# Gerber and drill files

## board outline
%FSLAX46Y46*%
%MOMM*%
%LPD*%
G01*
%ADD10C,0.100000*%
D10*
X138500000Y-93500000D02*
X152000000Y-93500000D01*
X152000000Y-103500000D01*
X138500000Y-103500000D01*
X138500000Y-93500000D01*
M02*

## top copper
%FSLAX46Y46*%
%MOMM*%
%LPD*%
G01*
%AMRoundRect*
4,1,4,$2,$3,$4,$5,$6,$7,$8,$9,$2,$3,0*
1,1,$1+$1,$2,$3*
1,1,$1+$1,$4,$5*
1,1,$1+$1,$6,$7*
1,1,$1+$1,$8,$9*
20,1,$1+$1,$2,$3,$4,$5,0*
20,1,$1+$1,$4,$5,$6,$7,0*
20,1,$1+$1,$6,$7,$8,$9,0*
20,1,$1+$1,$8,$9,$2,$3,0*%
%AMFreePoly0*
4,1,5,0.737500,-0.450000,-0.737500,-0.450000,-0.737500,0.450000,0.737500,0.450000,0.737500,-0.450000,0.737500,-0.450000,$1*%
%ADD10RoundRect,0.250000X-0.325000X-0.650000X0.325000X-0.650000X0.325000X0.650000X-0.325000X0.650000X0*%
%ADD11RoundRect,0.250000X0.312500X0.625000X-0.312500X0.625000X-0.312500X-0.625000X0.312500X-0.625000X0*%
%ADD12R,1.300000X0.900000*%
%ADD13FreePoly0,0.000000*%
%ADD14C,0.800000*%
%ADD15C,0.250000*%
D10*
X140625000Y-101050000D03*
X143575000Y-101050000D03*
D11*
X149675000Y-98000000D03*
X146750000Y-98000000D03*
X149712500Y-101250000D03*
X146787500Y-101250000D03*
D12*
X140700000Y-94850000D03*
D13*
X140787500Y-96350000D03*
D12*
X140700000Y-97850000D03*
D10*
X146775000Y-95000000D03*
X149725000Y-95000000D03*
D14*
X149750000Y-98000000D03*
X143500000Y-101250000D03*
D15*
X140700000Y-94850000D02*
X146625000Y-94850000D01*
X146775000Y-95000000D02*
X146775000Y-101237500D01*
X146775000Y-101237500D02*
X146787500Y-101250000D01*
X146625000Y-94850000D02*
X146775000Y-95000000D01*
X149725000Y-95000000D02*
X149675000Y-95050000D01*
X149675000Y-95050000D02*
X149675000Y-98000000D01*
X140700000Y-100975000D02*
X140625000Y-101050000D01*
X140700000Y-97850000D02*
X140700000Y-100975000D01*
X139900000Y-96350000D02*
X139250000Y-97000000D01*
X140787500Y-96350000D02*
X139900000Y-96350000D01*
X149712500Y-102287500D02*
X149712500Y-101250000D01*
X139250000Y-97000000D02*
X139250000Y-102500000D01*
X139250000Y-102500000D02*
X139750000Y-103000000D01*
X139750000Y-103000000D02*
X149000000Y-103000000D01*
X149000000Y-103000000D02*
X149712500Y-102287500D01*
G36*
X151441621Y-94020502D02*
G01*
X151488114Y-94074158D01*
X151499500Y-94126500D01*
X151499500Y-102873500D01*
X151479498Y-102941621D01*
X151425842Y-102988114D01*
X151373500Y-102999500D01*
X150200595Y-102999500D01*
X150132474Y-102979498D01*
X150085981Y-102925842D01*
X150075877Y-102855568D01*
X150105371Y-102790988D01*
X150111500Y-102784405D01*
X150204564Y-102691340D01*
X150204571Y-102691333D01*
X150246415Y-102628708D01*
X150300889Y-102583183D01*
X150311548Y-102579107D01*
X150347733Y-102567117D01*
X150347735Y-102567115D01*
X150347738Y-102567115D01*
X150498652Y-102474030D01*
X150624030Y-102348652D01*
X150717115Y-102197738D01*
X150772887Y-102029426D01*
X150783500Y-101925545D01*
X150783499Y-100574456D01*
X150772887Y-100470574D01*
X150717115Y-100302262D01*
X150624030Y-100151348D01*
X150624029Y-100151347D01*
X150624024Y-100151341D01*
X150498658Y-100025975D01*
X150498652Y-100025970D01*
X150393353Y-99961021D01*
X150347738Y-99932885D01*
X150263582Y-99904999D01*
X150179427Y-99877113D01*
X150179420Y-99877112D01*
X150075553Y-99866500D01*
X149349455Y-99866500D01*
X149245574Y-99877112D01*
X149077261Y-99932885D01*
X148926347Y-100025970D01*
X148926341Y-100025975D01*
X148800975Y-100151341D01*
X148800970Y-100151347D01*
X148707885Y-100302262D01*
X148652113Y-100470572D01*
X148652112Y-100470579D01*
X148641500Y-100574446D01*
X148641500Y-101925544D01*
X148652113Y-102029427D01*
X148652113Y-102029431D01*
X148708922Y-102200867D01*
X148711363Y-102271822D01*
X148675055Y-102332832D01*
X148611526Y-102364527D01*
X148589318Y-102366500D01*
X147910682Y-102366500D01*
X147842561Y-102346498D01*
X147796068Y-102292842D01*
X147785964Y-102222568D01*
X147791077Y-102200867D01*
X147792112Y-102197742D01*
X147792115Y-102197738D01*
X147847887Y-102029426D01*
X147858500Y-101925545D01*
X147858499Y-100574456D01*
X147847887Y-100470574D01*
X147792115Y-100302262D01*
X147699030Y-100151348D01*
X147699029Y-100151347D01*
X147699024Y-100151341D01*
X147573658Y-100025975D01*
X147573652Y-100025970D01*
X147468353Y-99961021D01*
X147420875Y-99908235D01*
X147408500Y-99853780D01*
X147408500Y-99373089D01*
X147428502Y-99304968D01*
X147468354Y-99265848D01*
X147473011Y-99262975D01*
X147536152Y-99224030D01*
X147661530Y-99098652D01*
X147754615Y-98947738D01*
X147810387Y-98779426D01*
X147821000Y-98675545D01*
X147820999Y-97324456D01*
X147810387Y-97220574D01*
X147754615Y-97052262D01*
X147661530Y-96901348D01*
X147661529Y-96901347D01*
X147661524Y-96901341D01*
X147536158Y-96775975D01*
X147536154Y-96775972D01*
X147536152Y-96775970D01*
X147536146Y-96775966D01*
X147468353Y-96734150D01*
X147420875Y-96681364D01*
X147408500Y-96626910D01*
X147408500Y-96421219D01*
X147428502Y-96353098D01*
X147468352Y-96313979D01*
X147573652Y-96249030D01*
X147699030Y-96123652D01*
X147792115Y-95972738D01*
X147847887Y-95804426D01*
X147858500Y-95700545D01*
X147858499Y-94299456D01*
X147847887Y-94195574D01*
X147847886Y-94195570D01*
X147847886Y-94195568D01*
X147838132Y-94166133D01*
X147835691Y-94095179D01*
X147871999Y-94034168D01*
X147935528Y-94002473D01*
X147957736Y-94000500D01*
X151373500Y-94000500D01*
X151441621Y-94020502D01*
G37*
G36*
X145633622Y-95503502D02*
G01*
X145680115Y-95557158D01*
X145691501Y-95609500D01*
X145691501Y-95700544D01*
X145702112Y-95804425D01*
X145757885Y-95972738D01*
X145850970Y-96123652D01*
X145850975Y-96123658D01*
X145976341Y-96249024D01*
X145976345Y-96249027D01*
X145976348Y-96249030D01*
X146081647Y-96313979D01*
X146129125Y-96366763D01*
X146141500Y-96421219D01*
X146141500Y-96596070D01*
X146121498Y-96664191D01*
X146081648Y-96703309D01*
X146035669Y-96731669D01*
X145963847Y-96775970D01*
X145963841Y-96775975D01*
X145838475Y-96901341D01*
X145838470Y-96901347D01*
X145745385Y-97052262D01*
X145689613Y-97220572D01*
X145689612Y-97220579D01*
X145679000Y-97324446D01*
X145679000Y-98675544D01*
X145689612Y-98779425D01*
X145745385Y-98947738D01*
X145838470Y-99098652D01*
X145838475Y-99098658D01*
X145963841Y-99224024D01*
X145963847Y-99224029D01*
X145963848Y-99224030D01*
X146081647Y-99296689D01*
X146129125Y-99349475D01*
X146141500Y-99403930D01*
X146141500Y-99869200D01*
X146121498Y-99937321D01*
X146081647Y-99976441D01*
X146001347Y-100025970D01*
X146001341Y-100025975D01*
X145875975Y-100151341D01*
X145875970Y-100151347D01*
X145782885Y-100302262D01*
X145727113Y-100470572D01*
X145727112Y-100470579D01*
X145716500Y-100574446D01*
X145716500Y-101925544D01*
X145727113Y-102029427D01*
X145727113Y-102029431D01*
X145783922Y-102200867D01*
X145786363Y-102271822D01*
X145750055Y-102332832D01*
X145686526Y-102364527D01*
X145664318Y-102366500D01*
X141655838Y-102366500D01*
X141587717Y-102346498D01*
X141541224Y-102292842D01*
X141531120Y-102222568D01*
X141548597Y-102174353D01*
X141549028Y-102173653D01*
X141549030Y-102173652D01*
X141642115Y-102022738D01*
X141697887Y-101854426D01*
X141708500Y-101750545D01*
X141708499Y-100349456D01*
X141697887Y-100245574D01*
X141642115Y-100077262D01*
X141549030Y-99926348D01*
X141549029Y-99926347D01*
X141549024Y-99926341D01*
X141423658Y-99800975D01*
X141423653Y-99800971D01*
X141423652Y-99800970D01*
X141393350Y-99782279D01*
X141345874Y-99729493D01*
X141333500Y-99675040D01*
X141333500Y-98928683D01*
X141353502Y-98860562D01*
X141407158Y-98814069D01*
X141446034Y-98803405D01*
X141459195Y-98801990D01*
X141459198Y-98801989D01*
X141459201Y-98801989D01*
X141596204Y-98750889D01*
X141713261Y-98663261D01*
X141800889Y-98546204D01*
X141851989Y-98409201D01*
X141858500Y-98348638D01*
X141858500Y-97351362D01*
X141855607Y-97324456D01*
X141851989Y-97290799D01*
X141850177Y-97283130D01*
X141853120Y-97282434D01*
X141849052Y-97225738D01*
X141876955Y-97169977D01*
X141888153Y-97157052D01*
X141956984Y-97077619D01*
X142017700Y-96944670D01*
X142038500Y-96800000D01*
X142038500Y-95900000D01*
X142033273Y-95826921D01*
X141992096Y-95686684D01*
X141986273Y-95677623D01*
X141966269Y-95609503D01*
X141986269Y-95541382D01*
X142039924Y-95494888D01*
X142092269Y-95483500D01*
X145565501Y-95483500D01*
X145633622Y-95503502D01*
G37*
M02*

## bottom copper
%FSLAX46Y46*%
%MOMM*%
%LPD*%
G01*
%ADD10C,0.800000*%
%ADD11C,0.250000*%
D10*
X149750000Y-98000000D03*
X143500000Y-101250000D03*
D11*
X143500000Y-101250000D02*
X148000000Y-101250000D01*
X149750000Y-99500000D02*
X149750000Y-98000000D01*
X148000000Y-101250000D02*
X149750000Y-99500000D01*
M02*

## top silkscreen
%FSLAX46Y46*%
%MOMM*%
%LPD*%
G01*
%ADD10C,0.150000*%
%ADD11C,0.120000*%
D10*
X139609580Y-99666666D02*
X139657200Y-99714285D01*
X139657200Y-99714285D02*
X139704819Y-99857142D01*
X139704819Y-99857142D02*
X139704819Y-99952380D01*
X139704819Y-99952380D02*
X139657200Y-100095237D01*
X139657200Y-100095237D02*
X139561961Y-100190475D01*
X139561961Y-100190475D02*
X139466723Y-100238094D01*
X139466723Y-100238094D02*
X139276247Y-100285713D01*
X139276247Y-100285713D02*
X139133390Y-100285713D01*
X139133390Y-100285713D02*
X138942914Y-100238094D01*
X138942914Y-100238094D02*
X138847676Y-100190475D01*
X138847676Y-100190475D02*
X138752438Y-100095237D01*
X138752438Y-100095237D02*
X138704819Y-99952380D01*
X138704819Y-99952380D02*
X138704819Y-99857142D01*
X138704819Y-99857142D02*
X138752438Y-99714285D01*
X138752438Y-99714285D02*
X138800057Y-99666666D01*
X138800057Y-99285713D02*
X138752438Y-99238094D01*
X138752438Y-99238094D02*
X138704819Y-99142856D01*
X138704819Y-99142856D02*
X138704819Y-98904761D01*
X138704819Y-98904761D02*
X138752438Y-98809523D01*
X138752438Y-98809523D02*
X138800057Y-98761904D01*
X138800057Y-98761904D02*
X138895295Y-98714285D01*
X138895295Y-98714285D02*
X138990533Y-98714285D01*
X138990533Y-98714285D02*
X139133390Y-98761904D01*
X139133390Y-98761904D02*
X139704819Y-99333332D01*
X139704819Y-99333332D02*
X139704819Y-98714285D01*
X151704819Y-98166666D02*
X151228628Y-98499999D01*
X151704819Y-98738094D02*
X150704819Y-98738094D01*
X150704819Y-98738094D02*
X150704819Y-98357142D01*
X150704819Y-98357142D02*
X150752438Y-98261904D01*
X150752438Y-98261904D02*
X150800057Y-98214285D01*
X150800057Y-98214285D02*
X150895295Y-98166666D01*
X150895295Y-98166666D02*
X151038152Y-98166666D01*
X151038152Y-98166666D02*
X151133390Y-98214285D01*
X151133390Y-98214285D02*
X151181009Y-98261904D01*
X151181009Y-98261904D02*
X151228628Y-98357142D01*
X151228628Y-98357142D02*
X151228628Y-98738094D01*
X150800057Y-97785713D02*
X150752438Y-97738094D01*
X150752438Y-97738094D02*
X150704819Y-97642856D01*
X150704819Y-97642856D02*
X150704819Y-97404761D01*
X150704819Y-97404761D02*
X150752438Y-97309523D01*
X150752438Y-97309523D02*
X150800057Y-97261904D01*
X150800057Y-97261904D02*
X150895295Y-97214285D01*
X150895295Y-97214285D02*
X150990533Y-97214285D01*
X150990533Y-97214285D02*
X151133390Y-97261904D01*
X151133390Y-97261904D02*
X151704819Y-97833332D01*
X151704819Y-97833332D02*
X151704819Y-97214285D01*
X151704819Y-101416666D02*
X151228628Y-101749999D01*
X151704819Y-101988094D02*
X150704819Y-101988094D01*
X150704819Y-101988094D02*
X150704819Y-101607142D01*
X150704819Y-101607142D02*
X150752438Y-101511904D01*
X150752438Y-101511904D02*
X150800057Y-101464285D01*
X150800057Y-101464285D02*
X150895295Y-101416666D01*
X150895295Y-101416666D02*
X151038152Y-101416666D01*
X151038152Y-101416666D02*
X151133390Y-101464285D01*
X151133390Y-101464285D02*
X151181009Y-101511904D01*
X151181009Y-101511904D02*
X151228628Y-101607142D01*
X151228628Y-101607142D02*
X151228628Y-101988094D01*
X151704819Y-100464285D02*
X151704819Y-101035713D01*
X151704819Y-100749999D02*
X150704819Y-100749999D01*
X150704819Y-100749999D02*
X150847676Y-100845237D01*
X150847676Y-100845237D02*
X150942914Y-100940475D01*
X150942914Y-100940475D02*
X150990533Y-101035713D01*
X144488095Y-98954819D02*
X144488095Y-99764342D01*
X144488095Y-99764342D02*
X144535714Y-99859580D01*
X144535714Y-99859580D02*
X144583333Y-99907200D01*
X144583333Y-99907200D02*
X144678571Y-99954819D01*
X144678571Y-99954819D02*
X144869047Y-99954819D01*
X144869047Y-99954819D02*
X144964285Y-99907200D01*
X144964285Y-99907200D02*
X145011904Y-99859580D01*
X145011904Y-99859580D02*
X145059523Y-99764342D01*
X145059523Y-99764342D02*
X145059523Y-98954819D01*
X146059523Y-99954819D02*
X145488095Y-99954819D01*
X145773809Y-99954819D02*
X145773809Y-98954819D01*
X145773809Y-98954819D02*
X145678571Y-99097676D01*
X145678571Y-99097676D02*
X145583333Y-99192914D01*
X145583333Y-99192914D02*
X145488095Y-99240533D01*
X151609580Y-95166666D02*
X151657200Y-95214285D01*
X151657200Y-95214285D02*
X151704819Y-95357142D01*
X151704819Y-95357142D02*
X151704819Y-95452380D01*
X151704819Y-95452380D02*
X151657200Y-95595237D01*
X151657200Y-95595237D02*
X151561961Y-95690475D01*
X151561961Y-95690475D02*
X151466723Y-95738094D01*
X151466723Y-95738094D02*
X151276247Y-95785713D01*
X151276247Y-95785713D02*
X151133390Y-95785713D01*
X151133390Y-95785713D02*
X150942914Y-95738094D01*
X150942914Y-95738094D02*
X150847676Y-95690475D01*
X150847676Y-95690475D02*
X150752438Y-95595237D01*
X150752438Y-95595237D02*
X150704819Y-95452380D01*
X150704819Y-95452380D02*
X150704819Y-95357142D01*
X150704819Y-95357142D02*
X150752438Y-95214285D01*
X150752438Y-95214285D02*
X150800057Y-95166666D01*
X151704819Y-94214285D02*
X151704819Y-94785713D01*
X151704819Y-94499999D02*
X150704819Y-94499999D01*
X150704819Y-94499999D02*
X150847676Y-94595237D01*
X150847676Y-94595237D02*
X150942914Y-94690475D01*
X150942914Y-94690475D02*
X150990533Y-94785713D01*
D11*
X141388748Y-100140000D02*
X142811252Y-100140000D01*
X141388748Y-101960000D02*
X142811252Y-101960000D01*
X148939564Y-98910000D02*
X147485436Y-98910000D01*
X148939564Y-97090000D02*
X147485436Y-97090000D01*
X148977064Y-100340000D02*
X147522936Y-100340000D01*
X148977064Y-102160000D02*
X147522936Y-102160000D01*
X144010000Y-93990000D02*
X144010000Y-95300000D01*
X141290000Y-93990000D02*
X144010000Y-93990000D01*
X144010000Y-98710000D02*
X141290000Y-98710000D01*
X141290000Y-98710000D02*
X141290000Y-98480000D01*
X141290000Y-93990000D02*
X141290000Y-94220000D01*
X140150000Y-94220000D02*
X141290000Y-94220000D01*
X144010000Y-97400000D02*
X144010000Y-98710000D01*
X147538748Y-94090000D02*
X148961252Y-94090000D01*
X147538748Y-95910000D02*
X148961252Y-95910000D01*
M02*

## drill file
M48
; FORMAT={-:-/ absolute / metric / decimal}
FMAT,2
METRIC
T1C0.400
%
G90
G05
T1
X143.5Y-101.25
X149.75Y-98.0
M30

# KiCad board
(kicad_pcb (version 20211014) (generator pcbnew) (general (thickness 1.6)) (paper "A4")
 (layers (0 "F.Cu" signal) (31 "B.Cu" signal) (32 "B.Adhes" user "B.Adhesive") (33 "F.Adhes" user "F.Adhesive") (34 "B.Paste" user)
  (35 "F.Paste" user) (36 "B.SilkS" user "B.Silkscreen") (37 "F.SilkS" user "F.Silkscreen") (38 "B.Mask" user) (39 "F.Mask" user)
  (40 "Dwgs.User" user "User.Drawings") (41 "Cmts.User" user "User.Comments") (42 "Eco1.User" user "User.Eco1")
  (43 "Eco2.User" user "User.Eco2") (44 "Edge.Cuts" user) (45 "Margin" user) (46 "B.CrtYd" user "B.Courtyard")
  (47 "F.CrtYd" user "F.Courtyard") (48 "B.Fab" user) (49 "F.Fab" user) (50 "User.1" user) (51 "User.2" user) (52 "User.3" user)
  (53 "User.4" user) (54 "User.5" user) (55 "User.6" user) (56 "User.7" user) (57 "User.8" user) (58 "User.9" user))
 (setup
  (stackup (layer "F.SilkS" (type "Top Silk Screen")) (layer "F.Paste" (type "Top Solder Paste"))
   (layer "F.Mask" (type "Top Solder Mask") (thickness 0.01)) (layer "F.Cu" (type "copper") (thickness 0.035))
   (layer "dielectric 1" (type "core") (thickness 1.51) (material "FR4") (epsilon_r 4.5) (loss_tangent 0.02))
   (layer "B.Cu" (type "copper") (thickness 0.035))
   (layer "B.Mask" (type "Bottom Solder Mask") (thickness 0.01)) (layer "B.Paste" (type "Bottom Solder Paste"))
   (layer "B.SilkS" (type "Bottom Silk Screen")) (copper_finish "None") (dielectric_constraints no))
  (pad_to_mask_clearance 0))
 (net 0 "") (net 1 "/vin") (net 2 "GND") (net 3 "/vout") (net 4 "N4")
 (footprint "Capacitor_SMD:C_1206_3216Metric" (layer "F.Cu") (at 142.1 101.05)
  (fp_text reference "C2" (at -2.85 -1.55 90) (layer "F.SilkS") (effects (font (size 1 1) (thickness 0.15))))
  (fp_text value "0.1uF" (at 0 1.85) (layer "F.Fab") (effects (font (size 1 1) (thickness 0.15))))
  (fp_line (start -0.711252 -0.91) (end 0.711252 -0.91) (layer "F.SilkS") (width 0.12))
  (fp_line (start -0.711252 0.91) (end 0.711252 0.91) (layer "F.SilkS") (width 0.12))
  (pad "1" smd roundrect (at -1.475 0) (size 1.15 1.8) (layers "F.Cu" "F.Paste" "F.Mask") (roundrect_rratio 0.2173913043) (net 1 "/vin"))
  (pad "2" smd roundrect (at 1.475 0) (size 1.15 1.8) (layers "F.Cu" "F.Paste" "F.Mask") (roundrect_rratio 0.2173913043) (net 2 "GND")))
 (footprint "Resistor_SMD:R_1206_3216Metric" (layer "F.Cu") (at 148.2125 98 180)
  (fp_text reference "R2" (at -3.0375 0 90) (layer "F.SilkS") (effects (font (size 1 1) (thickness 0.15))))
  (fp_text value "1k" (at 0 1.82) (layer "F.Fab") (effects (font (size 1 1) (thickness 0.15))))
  (fp_line (start -0.727064 -0.91) (end 0.727064 -0.91) (layer "F.SilkS") (width 0.12))
  (fp_line (start -0.727064 0.91) (end 0.727064 0.91) (layer "F.SilkS") (width 0.12))
  (pad "1" smd roundrect (at -1.4625 0 180) (size 1.125 1.75) (layers "F.Cu" "F.Paste" "F.Mask") (roundrect_rratio 0.2222222222)
   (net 2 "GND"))
  (pad "2" smd roundrect (at 1.4625 0 180) (size 1.125 1.75) (layers "F.Cu" "F.Paste" "F.Mask") (roundrect_rratio 0.2222222222)
   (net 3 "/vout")))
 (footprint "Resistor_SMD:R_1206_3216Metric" (layer "F.Cu") (at 148.25 101.25 180)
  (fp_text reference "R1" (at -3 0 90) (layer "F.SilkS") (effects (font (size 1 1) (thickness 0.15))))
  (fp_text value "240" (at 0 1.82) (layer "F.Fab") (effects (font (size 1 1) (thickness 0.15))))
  (fp_line (start -0.727064 0.91) (end 0.727064 0.91) (layer "F.SilkS") (width 0.12))
  (fp_line (start -0.727064 -0.91) (end 0.727064 -0.91) (layer "F.SilkS") (width 0.12))
  (pad "1" smd roundrect (at -1.4625 0 180) (size 1.125 1.75) (layers "F.Cu" "F.Paste" "F.Mask") (roundrect_rratio 0.2222222222)
   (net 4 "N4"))
  (pad "2" smd roundrect (at 1.4625 0 180) (size 1.125 1.75) (layers "F.Cu" "F.Paste" "F.Mask") (roundrect_rratio 0.2222222222)
   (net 3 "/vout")))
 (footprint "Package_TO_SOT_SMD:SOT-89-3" (layer "F.Cu") (at 142.35 96.35)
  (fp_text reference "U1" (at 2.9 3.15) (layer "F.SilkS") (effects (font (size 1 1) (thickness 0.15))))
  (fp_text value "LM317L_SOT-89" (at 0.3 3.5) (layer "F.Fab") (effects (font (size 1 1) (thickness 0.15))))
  (fp_line (start 1.66 -2.36) (end 1.66 -1.05) (layer "F.SilkS") (width 0.12))
  (fp_line (start -1.06 -2.36) (end 1.66 -2.36) (layer "F.SilkS") (width 0.12))
  (fp_line (start 1.66 2.36) (end -1.06 2.36) (layer "F.SilkS") (width 0.12))
  (fp_line (start -1.06 2.36) (end -1.06 2.13) (layer "F.SilkS") (width 0.12))
  (fp_line (start -1.06 -2.36) (end -1.06 -2.13) (layer "F.SilkS") (width 0.12))
  (fp_line (start -2.2 -2.13) (end -1.06 -2.13) (layer "F.SilkS") (width 0.12))
  (fp_line (start 1.66 1.05) (end 1.66 2.36) (layer "F.SilkS") (width 0.12))
  (pad "1" smd rect (at -1.65 -1.5) (size 1.3 0.9) (layers "F.Cu" "F.Paste" "F.Mask") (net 3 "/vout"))
  (pad "2" smd custom (at -1.5625 0) (size 1.475 0.9) (layers "F.Cu" "F.Paste" "F.Mask") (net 4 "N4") (zone_connect 2)
   (options (clearance outline) (anchor rect)) (primitives))
  (pad "3" smd rect (at -1.65 1.5) (size 1.3 0.9) (layers "F.Cu" "F.Paste" "F.Mask") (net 1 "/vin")))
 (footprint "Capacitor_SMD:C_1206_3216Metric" (layer "F.Cu") (at 148.25 95)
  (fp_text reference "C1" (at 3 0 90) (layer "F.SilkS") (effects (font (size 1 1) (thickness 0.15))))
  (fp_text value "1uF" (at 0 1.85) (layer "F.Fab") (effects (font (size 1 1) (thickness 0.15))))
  (fp_line (start -0.711252 -0.91) (end 0.711252 -0.91) (layer "F.SilkS") (width 0.12))
  (fp_line (start -0.711252 0.91) (end 0.711252 0.91) (layer "F.SilkS") (width 0.12))
  (pad "1" smd roundrect (at -1.475 0) (size 1.15 1.8) (layers "F.Cu" "F.Paste" "F.Mask") (roundrect_rratio 0.2173913043) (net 3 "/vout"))
  (pad "2" smd roundrect (at 1.475 0) (size 1.15 1.8) (layers "F.Cu" "F.Paste" "F.Mask") (roundrect_rratio 0.2173913043) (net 2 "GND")))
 (gr_rect (start 138.5 93.5) (end 152 103.5) (layer "Edge.Cuts") (width 0.1) (fill none))
 (segment (start 140.7 94.85) (end 146.625 94.85) (width 0.25) (layer "F.Cu") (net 3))
 (segment (start 146.775 95) (end 146.775 101.2375) (width 0.25) (layer "F.Cu") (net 3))
 (segment (start 146.775 101.2375) (end 146.7875 101.25) (width 0.25) (layer "F.Cu") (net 3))
 (segment (start 146.625 94.85) (end 146.775 95) (width 0.25) (layer "F.Cu") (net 3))
 (segment (start 149.725 95) (end 149.675 95.05) (width 0.25) (layer "F.Cu") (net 2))
 (segment (start 149.675 95.05) (end 149.675 98) (width 0.25) (layer "F.Cu") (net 2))
 (via (at 149.75 98) (size 0.8) (drill 0.4) (layers "F.Cu" "B.Cu") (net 2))
 (via (at 143.5 101.25) (size 0.8) (drill 0.4) (layers "F.Cu" "B.Cu") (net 2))
 (segment (start 143.5 101.25) (end 148 101.25) (width 0.25) (layer "B.Cu") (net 2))
 (segment (start 149.75 99.5) (end 149.75 98) (width 0.25) (layer "B.Cu") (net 2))
 (segment (start 148 101.25) (end 149.75 99.5) (width 0.25) (layer "B.Cu") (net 2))
 (segment (start 140.7 100.975) (end 140.625 101.05) (width 0.25) (layer "F.Cu") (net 1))
 (segment (start 140.7 97.85) (end 140.7 100.975) (width 0.25) (layer "F.Cu") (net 1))
 (segment (start 139.9 96.35) (end 139.25 97) (width 0.25) (layer "F.Cu") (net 4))
 (segment (start 140.7875 96.35) (end 139.9 96.35) (width 0.25) (layer "F.Cu") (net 4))
 (segment (start 149.7125 102.2875) (end 149.7125 101.25) (width 0.25) (layer "F.Cu") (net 4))
 (segment (start 139.25 97) (end 139.25 102.5) (width 0.25) (layer "F.Cu") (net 4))
 (segment (start 139.25 102.5) (end 139.75 103) (width 0.25) (layer "F.Cu") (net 4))
 (segment (start 139.75 103) (end 149 103) (width 0.25) (layer "F.Cu") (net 4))
 (segment (start 149 103) (end 149.7125 102.2875) (width 0.25) (layer "F.Cu") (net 4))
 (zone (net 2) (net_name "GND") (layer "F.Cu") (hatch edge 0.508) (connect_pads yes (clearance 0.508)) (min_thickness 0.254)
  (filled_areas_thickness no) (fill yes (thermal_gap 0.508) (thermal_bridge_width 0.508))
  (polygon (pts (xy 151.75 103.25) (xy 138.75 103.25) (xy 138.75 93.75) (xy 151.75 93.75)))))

